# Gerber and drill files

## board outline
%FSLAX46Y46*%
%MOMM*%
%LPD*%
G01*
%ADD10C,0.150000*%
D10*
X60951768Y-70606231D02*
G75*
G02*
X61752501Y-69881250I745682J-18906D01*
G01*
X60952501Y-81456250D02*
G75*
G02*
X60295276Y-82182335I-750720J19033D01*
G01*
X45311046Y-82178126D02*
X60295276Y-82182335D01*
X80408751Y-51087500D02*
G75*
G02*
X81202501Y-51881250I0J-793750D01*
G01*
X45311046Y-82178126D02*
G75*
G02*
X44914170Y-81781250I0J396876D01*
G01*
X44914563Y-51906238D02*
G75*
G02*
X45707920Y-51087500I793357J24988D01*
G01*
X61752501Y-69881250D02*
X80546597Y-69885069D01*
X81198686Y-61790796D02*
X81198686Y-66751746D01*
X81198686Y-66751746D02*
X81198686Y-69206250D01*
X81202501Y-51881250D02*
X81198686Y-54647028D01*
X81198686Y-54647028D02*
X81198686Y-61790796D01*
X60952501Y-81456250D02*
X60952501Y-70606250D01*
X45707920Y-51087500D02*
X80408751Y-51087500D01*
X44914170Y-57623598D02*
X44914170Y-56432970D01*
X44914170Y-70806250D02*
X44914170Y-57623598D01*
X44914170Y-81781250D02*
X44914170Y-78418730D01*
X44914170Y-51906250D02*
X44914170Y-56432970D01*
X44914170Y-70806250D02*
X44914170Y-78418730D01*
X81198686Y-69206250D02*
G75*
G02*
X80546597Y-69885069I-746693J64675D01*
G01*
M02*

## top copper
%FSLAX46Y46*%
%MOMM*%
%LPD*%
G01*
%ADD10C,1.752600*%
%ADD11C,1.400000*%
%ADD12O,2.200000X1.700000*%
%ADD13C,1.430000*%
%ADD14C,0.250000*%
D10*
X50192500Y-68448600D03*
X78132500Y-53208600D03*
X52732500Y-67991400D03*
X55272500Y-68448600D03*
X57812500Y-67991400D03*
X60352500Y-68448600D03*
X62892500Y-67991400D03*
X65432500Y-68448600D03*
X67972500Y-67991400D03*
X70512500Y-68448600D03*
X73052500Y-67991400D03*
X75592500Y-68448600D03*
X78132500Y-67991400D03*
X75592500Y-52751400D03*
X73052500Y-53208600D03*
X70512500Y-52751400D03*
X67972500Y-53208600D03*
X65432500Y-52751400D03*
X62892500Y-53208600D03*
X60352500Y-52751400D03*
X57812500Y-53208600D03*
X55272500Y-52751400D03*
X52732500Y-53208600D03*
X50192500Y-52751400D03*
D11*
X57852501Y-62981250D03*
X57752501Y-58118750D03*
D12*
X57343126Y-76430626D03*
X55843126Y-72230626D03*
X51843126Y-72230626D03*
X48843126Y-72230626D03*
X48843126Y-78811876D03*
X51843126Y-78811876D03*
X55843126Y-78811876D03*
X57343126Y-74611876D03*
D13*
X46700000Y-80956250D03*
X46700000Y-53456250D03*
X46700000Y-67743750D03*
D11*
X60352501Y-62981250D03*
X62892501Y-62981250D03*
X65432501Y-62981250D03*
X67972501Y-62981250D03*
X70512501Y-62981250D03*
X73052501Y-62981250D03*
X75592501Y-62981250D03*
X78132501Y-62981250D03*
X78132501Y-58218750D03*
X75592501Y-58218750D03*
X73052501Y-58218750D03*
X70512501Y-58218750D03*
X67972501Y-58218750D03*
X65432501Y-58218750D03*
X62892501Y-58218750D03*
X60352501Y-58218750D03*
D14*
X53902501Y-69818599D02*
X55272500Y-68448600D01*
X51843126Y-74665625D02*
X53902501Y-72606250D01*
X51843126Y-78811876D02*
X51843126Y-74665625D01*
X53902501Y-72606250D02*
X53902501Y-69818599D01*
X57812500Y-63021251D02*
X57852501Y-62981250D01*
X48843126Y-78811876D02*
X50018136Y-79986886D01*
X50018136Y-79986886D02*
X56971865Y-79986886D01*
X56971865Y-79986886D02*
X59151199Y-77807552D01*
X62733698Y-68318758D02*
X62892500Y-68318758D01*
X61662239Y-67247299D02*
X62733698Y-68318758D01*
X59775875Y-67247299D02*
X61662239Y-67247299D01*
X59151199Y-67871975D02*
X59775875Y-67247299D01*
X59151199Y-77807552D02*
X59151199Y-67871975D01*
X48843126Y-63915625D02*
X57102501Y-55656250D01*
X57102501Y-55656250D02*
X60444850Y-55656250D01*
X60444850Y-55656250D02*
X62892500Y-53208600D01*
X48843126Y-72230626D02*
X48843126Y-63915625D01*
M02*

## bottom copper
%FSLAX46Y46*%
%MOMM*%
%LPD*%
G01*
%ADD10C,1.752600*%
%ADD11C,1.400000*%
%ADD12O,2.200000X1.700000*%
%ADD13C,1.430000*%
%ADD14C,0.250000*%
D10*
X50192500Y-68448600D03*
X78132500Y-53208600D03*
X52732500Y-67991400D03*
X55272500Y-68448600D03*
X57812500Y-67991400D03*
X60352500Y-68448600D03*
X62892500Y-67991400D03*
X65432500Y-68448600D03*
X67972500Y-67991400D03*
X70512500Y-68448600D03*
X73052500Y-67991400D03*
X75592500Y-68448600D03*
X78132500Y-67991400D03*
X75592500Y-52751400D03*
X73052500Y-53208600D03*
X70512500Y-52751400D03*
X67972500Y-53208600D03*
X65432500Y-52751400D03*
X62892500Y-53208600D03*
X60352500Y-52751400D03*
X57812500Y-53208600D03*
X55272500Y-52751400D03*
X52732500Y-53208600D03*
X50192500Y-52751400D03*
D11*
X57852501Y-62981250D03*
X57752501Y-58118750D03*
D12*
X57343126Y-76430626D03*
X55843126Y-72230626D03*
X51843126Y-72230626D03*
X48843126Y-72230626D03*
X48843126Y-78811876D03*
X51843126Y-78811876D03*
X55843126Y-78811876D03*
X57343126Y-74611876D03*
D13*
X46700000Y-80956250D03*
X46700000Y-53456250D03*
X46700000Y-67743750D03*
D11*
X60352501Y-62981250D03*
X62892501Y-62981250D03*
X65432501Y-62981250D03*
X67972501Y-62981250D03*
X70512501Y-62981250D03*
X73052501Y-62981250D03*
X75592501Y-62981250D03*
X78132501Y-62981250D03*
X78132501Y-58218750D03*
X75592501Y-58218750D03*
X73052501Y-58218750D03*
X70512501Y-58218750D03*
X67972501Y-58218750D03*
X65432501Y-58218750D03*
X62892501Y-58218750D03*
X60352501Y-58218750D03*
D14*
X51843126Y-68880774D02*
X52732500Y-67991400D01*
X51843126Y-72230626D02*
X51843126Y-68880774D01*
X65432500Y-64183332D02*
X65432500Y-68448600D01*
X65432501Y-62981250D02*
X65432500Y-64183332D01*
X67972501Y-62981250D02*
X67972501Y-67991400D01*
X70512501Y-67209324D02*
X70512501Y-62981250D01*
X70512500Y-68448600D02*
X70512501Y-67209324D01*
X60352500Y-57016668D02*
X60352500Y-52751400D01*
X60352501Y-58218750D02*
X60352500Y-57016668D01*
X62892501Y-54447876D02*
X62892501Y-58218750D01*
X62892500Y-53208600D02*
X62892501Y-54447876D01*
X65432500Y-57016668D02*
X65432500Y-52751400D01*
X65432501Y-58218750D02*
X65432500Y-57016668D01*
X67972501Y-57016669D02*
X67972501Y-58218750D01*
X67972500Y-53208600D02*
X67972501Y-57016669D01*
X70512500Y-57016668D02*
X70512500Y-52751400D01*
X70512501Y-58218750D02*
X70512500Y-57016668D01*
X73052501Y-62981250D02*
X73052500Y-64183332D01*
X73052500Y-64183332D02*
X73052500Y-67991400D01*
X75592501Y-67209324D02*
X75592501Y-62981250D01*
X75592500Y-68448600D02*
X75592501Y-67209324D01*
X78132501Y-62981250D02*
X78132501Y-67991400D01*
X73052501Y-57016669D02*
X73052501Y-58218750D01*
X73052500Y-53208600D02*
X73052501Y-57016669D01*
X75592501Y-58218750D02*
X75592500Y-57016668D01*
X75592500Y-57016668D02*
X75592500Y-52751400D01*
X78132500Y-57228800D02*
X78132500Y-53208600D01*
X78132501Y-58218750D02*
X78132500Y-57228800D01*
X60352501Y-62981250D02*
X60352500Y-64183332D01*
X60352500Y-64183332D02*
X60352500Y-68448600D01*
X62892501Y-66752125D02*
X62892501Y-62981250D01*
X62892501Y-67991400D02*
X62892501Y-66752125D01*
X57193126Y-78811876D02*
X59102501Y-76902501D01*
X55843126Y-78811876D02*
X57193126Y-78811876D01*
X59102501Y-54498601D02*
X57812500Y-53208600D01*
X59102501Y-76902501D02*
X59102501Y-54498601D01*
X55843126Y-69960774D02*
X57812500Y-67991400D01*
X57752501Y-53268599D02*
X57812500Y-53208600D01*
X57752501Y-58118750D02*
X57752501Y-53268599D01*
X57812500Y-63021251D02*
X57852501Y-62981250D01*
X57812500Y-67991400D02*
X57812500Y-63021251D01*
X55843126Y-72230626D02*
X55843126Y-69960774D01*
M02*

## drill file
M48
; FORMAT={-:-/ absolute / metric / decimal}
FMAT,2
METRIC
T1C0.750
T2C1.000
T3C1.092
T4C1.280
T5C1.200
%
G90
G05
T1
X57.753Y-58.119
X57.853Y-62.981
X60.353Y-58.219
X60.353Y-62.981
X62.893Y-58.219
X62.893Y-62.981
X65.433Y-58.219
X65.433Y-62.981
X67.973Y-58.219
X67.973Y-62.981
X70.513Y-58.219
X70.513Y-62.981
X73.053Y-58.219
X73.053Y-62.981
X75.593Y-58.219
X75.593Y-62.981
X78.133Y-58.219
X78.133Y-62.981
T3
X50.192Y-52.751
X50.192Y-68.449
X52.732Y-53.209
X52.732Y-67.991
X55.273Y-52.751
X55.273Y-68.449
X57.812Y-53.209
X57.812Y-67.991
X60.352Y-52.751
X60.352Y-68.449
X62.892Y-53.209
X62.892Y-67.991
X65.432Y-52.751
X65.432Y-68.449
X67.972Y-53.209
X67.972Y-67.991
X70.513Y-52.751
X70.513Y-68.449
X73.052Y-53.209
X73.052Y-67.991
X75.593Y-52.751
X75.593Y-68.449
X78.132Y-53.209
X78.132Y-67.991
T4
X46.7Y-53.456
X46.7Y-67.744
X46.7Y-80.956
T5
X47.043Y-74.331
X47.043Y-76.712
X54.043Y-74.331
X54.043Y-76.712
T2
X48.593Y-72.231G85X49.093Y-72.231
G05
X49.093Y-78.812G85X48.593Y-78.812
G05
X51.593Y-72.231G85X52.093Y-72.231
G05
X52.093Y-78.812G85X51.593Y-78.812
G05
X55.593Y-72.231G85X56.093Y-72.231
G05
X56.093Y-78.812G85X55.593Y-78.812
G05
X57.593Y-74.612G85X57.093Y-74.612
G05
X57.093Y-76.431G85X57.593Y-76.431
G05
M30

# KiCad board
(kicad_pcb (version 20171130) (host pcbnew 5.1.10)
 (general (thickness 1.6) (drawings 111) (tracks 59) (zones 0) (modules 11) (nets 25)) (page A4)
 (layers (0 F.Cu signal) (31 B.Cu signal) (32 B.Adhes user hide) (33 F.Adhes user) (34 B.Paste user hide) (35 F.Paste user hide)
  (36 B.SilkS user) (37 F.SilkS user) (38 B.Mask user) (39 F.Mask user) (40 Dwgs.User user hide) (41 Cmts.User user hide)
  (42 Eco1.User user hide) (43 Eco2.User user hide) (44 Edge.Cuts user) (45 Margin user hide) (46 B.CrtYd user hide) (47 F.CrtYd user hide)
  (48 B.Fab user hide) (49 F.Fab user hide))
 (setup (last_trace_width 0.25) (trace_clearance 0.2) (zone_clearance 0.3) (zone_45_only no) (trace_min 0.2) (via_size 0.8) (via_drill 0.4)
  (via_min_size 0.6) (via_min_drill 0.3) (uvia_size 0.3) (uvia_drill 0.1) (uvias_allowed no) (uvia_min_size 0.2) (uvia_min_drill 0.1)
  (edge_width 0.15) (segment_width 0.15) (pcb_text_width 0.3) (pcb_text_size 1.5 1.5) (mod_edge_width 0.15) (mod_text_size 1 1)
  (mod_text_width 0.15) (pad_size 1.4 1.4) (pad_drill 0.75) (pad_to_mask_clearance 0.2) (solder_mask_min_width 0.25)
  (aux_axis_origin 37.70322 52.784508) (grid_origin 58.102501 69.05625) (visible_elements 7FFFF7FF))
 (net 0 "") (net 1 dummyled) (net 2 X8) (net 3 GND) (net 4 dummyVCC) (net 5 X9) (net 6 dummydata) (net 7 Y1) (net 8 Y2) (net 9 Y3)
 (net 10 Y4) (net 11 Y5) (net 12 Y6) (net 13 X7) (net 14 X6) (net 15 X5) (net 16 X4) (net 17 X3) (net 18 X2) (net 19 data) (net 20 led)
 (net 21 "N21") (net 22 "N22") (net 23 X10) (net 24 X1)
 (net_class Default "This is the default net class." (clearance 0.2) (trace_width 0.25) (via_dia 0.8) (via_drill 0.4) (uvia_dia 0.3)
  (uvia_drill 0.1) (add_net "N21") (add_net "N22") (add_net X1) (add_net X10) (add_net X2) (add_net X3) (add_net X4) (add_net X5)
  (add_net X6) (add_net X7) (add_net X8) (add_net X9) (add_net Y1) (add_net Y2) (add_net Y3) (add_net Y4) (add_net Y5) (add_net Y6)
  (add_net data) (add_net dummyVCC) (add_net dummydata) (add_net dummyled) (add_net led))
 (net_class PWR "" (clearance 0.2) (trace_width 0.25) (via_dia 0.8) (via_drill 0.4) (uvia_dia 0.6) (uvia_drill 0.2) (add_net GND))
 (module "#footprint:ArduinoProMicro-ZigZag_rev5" (layer B.Cu) (at 64.1625 60.6)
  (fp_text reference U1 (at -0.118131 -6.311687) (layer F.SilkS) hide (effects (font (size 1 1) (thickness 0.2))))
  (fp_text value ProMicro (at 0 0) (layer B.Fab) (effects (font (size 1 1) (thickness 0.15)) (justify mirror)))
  (pad 24 thru_hole circle (at -13.97 7.8486) (size 1.7526 1.7526) (drill 1.0922) (layers *.Cu *.SilkS *.Mask) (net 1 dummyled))
  (pad 12 thru_hole circle (at 13.97 -7.3914) (size 1.7526 1.7526) (drill 1.0922) (layers *.Cu *.SilkS *.Mask) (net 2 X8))
  (pad 23 thru_hole circle (at -11.43 7.3914) (size 1.7526 1.7526) (drill 1.0922) (layers *.Cu *.SilkS *.Mask) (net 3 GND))
  (pad 22 thru_hole circle (at -8.89 7.8486) (size 1.7526 1.7526) (drill 1.0922) (layers *.Cu *.SilkS *.Mask) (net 3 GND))
  (pad 21 thru_hole circle (at -6.35 7.3914) (size 1.7526 1.7526) (drill 1.0922) (layers *.Cu *.SilkS *.Mask) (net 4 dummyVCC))
  (pad 20 thru_hole circle (at -3.81 7.8486) (size 1.7526 1.7526) (drill 1.0922) (layers *.Cu *.SilkS *.Mask) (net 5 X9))
  (pad 19 thru_hole circle (at -1.27 7.3914) (size 1.7526 1.7526) (drill 1.0922) (layers *.Cu *.SilkS *.Mask) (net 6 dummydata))
  (pad 18 thru_hole circle (at 1.27 7.8486) (size 1.7526 1.7526) (drill 1.0922) (layers *.Cu *.SilkS *.Mask) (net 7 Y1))
  (pad 17 thru_hole circle (at 3.81 7.3914) (size 1.7526 1.7526) (drill 1.0922) (layers *.Cu *.SilkS *.Mask) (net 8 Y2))
  (pad 16 thru_hole circle (at 6.35 7.8486) (size 1.7526 1.7526) (drill 1.0922) (layers *.Cu *.SilkS *.Mask) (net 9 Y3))
  (pad 15 thru_hole circle (at 8.89 7.3914) (size 1.7526 1.7526) (drill 1.0922) (layers *.Cu *.SilkS *.Mask) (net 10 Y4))
  (pad 14 thru_hole circle (at 11.43 7.8486) (size 1.7526 1.7526) (drill 1.0922) (layers *.Cu *.SilkS *.Mask) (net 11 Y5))
  (pad 13 thru_hole circle (at 13.97 7.3914) (size 1.7526 1.7526) (drill 1.0922) (layers *.Cu *.SilkS *.Mask) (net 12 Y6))
  (pad 11 thru_hole circle (at 11.43 -7.8486) (size 1.7526 1.7526) (drill 1.0922) (layers *.Cu *.SilkS *.Mask) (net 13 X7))
  (pad 10 thru_hole circle (at 8.89 -7.3914) (size 1.7526 1.7526) (drill 1.0922) (layers *.Cu *.SilkS *.Mask) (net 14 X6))
  (pad 9 thru_hole circle (at 6.35 -7.8486) (size 1.7526 1.7526) (drill 1.0922) (layers *.Cu *.SilkS *.Mask) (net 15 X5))
  (pad 8 thru_hole circle (at 3.81 -7.3914) (size 1.7526 1.7526) (drill 1.0922) (layers *.Cu *.SilkS *.Mask) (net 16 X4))
  (pad 7 thru_hole circle (at 1.27 -7.8486) (size 1.7526 1.7526) (drill 1.0922) (layers *.Cu *.SilkS *.Mask) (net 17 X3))
  (pad 6 thru_hole circle (at -1.27 -7.3914) (size 1.7526 1.7526) (drill 1.0922) (layers *.Cu *.SilkS *.Mask) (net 6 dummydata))
  (pad 5 thru_hole circle (at -3.81 -7.8486) (size 1.7526 1.7526) (drill 1.0922) (layers *.Cu *.SilkS *.Mask) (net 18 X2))
  (pad 4 thru_hole circle (at -6.35 -7.3914) (size 1.7526 1.7526) (drill 1.0922) (layers *.Cu *.SilkS *.Mask) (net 4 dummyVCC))
  (pad 3 thru_hole circle (at -8.89 -7.8486) (size 1.7526 1.7526) (drill 1.0922) (layers *.Cu *.SilkS *.Mask) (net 3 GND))
  (pad 2 thru_hole circle (at -11.43 -7.3914) (size 1.7526 1.7526) (drill 1.0922) (layers *.Cu *.SilkS *.Mask) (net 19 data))
  (pad 1 thru_hole circle (at -13.97 -7.8486) (size 1.7526 1.7526) (drill 1.0922) (layers *.Cu *.SilkS *.Mask) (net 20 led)))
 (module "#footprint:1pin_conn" (layer F.Cu) (at 57.852501 63.00625) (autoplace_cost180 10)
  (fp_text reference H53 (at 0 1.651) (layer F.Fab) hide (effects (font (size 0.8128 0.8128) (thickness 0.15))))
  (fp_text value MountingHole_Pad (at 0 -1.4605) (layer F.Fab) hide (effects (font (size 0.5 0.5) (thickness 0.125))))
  (pad 1 thru_hole circle (at 0 -0.025) (size 1.4 1.4) (drill 0.75) (layers *.Cu *.Mask) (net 4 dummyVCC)))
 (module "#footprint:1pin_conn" (layer F.Cu) (at 57.752501 58.21875) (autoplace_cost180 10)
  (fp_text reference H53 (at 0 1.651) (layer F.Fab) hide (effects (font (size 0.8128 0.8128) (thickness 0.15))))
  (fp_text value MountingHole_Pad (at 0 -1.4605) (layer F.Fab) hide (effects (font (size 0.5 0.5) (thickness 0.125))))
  (pad 1 thru_hole circle (at 0 -0.1) (size 1.4 1.4) (drill 0.75) (layers *.Cu *.Mask) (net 4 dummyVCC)))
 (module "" (layer F.Cu) (at 7.352501 -16.34375)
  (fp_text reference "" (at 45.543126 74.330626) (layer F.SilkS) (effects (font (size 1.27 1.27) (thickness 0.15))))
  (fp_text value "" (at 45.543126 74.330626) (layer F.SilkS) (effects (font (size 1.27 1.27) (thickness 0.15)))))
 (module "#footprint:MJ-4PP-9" (layer F.Cu) (at 45.543126 74.330626 90)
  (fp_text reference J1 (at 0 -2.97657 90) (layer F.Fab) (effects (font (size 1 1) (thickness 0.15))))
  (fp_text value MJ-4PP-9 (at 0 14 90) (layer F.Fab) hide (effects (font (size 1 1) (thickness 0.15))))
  (pad A thru_hole oval (at -2.1 11.8 90) (size 1.7 2.2) (drill oval 1 1.5) (layers *.Cu *.Mask F.SilkS) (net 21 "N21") (clearance 0.15))
  (pad D thru_hole oval (at 2.1 10.3 90) (size 1.7 2.2) (drill oval 1 1.5) (layers *.Cu *.Mask F.SilkS) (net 4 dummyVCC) (clearance 0.15))
  (pad C thru_hole oval (at 2.1 6.3 90) (size 1.7 2.2) (drill oval 1 1.5) (layers *.Cu *.Mask F.SilkS) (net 3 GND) (clearance 0.15))
  (pad B thru_hole oval (at 2.1 3.3 90) (size 1.7 2.2) (drill oval 1 1.5) (layers *.Cu *.Mask F.SilkS) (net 6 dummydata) (clearance 0.15))
  (pad "" np_thru_hole circle (at 0 8.5 90) (size 1.2 1.2) (drill 1.2) (layers *.Cu *.Mask F.SilkS))
  (pad "" np_thru_hole circle (at 0 1.5 90) (size 1.2 1.2) (drill 1.2) (layers *.Cu *.Mask F.SilkS)))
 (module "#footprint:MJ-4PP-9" (layer B.Cu) (at 45.543126 76.711876 270)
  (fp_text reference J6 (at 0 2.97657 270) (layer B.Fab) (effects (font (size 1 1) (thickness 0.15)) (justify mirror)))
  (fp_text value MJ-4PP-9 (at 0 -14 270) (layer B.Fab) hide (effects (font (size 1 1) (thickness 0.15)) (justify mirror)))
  (pad "" np_thru_hole circle (at 0 -1.5 270) (size 1.2 1.2) (drill 1.2) (layers *.Cu *.Mask B.SilkS))
  (pad "" np_thru_hole circle (at 0 -8.5 270) (size 1.2 1.2) (drill 1.2) (layers *.Cu *.Mask B.SilkS))
  (pad B thru_hole oval (at 2.1 -3.3 270) (size 1.7 2.2) (drill oval 1 1.5) (layers *.Cu *.Mask B.SilkS) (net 6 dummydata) (clearance 0.15))
  (pad C thru_hole oval (at 2.1 -6.3 270) (size 1.7 2.2) (drill oval 1 1.5) (layers *.Cu *.Mask B.SilkS) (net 3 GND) (clearance 0.15))
  (pad D thru_hole oval (at 2.1 -10.3 270) (size 1.7 2.2) (drill oval 1 1.5) (layers *.Cu *.Mask B.SilkS) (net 4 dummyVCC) (clearance 0.15))
  (pad A thru_hole oval (at -2.1 -11.8 270) (size 1.7 2.2) (drill oval 1 1.5) (layers *.Cu *.Mask B.SilkS) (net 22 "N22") (clearance 0.15)))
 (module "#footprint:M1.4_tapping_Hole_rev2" (layer F.Cu) (at 46.102501 80.95625) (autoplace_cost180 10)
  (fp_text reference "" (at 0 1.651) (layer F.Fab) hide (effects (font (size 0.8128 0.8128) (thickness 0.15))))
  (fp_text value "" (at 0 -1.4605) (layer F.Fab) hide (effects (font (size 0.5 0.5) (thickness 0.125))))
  (pad "" thru_hole circle (at 0.597499 0) (size 1.43 1.43) (drill 1.28) (layers *.Cu *.Mask)))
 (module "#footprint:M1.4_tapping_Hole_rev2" (layer F.Cu) (at 46.7 53.45625) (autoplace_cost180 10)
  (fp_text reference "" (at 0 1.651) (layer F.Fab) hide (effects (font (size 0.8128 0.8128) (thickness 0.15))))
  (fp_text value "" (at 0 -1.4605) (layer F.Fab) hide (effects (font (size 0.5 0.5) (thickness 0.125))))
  (pad "" thru_hole circle (at 0 0) (size 1.43 1.43) (drill 1.28) (layers *.Cu *.Mask)))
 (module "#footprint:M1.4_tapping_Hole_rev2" (layer F.Cu) (at 46.7 67.74375) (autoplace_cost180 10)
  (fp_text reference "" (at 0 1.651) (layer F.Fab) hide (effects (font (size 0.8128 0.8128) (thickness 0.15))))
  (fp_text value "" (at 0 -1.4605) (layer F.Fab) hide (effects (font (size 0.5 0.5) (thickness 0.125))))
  (pad "" thru_hole circle (at 0 0) (size 1.43 1.43) (drill 1.28) (layers *.Cu *.Mask)))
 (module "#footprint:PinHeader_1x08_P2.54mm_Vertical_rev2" (layer F.Cu) (at 60.352501 62.98125 90)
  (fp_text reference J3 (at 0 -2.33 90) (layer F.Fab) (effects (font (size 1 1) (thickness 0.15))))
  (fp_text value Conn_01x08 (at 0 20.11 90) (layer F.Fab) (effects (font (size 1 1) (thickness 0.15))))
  (pad 1 thru_hole circle (at 0 0 90) (size 1.4 1.4) (drill 0.75) (layers *.Cu *.Mask) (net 5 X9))
  (pad 2 thru_hole circle (at 0 2.54 90) (size 1.4 1.4) (drill 0.75) (layers *.Cu *.Mask) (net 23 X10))
  (pad 3 thru_hole circle (at 0 5.08 90) (size 1.4 1.4) (drill 0.75) (layers *.Cu *.Mask) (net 7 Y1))
  (pad 4 thru_hole circle (at 0 7.62 90) (size 1.4 1.4) (drill 0.75) (layers *.Cu *.Mask) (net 8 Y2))
  (pad 5 thru_hole circle (at 0 10.16 90) (size 1.4 1.4) (drill 0.75) (layers *.Cu *.Mask) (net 9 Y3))
  (pad 6 thru_hole circle (at 0 12.7 90) (size 1.4 1.4) (drill 0.75) (layers *.Cu *.Mask) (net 10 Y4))
  (pad 7 thru_hole circle (at 0 15.24 90) (size 1.4 1.4) (drill 0.75) (layers *.Cu *.Mask) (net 11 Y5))
  (pad 8 thru_hole circle (at 0 17.78 90) (size 1.4 1.4) (drill 0.75) (layers *.Cu *.Mask) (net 12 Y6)))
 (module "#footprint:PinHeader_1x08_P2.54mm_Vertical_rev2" (layer F.Cu) (at 60.352501 58.21875 90)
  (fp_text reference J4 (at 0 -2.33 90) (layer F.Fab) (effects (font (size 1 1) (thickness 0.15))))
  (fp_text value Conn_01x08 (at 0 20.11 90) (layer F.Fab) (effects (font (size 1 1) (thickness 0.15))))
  (pad 8 thru_hole circle (at 0 17.78 90) (size 1.4 1.4) (drill 0.75) (layers *.Cu *.Mask) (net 2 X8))
  (pad 7 thru_hole circle (at 0 15.24 90) (size 1.4 1.4) (drill 0.75) (layers *.Cu *.Mask) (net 13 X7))
  (pad 6 thru_hole circle (at 0 12.7 90) (size 1.4 1.4) (drill 0.75) (layers *.Cu *.Mask) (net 14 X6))
  (pad 5 thru_hole circle (at 0 10.16 90) (size 1.4 1.4) (drill 0.75) (layers *.Cu *.Mask) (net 15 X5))
  (pad 4 thru_hole circle (at 0 7.62 90) (size 1.4 1.4) (drill 0.75) (layers *.Cu *.Mask) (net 16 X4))
  (pad 3 thru_hole circle (at 0 5.08 90) (size 1.4 1.4) (drill 0.75) (layers *.Cu *.Mask) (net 17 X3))
  (pad 2 thru_hole circle (at 0 2.54 90) (size 1.4 1.4) (drill 0.75) (layers *.Cu *.Mask) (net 18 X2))
  (pad 1 thru_hole circle (at 0 0 90) (size 1.4 1.4) (drill 0.75) (layers *.Cu *.Mask) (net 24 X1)))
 (gr_arc (start 61.69745 70.625137) (end 61.752501 69.88125) (angle -92.78006695) (layer Edge.Cuts) (width 0.15))
 (gr_arc (start 60.201781 81.437217) (end 60.295276 82.182335) (angle -81.39578011) (layer Edge.Cuts) (width 0.15))
 (gr_line (start 45.311046 82.178126) (end 60.295276 82.182335) (layer Edge.Cuts) (width 0.15))
 (gr_arc (start 80.408751 51.88125) (end 81.202501 51.88125) (angle -90) (layer Edge.Cuts) (width 0.15))
 (gr_arc (start 45.311046 81.78125) (end 44.91417 81.78125) (angle -90) (layer Edge.Cuts) (width 0.15))
 (gr_arc (start 45.70792 51.88125) (end 45.70792 51.0875) (angle -91.80399512) (layer Edge.Cuts) (width 0.15))
 (gr_line (start 61.752501 69.88125) (end 80.546597 69.885069) (layer Edge.Cuts) (width 0.15))
 (gr_line (start 81.198686 61.790796) (end 81.198686 66.751746) (layer Edge.Cuts) (width 0.15))
 (gr_line (start 81.198686 66.751746) (end 81.198686 69.20625) (layer Edge.Cuts) (width 0.15))
 (gr_line (start 81.202501 51.88125) (end 81.198686 54.647028) (layer Edge.Cuts) (width 0.15))
 (gr_line (start 81.198686 54.647028) (end 81.198686 61.790796) (layer Edge.Cuts) (width 0.15))
 (gr_line (start 60.952501 81.45625) (end 60.952501 70.60625) (layer Edge.Cuts) (width 0.15))
 (gr_line (start 45.70792 51.0875) (end 80.408751 51.0875) (layer Edge.Cuts) (width 0.15))
 (gr_line (start 44.91417 57.623598) (end 44.91417 56.43297) (layer Edge.Cuts) (width 0.15))
 (gr_line (start 44.91417 70.80625) (end 44.91417 57.623598) (layer Edge.Cuts) (width 0.15))
 (gr_line (start 44.91417 81.78125) (end 44.91417 78.41873) (layer Edge.Cuts) (width 0.15))
 (gr_line (start 44.91417 51.90625) (end 44.91417 56.43297) (layer Edge.Cuts) (width 0.15))
 (gr_line (start 44.91417 70.80625) (end 44.91417 78.41873) (layer Edge.Cuts) (width 0.15))
 (gr_arc (start 80.451993 69.141575) (end 80.546597 69.885069) (angle -77.79817896) (layer Edge.Cuts) (width 0.15))
 (segment (start 53.902501 69.818599) (end 55.2725 68.4486) (width 0.25) (layer F.Cu) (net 3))
 (segment (start 51.843126 74.665625) (end 53.902501 72.60625) (width 0.25) (layer F.Cu) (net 3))
 (segment (start 51.843126 78.811876) (end 51.843126 74.665625) (width 0.25) (layer F.Cu) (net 3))
 (segment (start 51.843126 68.880774) (end 52.7325 67.9914) (width 0.25) (layer B.Cu) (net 3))
 (segment (start 51.843126 72.230626) (end 51.843126 68.880774) (width 0.25) (layer B.Cu) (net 3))
 (segment (start 53.902501 72.60625) (end 53.902501 69.818599) (width 0.25) (layer F.Cu) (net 3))
 (segment (start 65.4325 64.183332) (end 65.4325 68.4486) (width 0.25) (layer B.Cu) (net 7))
 (segment (start 65.432501 62.98125) (end 65.4325 64.183332) (width 0.25) (layer B.Cu) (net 7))
 (segment (start 67.972501 62.98125) (end 67.972501 67.9914) (width 0.25) (layer B.Cu) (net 8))
 (segment (start 70.512501 67.209324) (end 70.512501 62.98125) (width 0.25) (layer B.Cu) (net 9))
 (segment (start 70.5125 68.4486) (end 70.512501 67.209324) (width 0.25) (layer B.Cu) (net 9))
 (segment (start 60.3525 57.016668) (end 60.3525 52.7514) (width 0.25) (layer B.Cu) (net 24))
 (segment (start 60.352501 58.21875) (end 60.3525 57.016668) (width 0.25) (layer B.Cu) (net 24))
 (segment (start 62.892501 54.447876) (end 62.892501 58.21875) (width 0.25) (layer B.Cu) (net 18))
 (segment (start 62.8925 53.2086) (end 62.892501 54.447876) (width 0.25) (layer B.Cu) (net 18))
 (segment (start 65.4325 57.016668) (end 65.4325 52.7514) (width 0.25) (layer B.Cu) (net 17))
 (segment (start 65.432501 58.21875) (end 65.4325 57.016668) (width 0.25) (layer B.Cu) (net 17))
 (segment (start 67.972501 57.016669) (end 67.972501 58.21875) (width 0.25) (layer B.Cu) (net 16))
 (segment (start 67.9725 53.2086) (end 67.972501 57.016669) (width 0.25) (layer B.Cu) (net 16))
 (segment (start 70.5125 57.016668) (end 70.5125 52.7514) (width 0.25) (layer B.Cu) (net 15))
 (segment (start 70.512501 58.21875) (end 70.5125 57.016668) (width 0.25) (layer B.Cu) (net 15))
 (segment (start 73.052501 62.98125) (end 73.0525 64.183332) (width 0.25) (layer B.Cu) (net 10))
 (segment (start 73.0525 64.183332) (end 73.0525 67.9914) (width 0.25) (layer B.Cu) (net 10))
 (segment (start 75.592501 67.209324) (end 75.592501 62.98125) (width 0.25) (layer B.Cu) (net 11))
 (segment (start 75.5925 68.4486) (end 75.592501 67.209324) (width 0.25) (layer B.Cu) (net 11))
 (segment (start 78.132501 62.98125) (end 78.132501 67.9914) (width 0.25) (layer B.Cu) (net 12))
 (segment (start 73.052501 57.016669) (end 73.052501 58.21875) (width 0.25) (layer B.Cu) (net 14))
 (segment (start 73.0525 53.2086) (end 73.052501 57.016669) (width 0.25) (layer B.Cu) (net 14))
 (segment (start 75.592501 58.21875) (end 75.5925 57.016668) (width 0.25) (layer B.Cu) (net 13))
 (segment (start 75.5925 57.016668) (end 75.5925 52.7514) (width 0.25) (layer B.Cu) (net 13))
 (segment (start 78.1325 57.2288) (end 78.1325 53.2086) (width 0.25) (layer B.Cu) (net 2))
 (segment (start 78.132501 58.21875) (end 78.1325 57.2288) (width 0.25) (layer B.Cu) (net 2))
 (segment (start 60.352501 62.98125) (end 60.3525 64.183332) (width 0.25) (layer B.Cu) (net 5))
 (segment (start 60.3525 64.183332) (end 60.3525 68.4486) (width 0.25) (layer B.Cu) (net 5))
 (segment (start 62.892501 66.752125) (end 62.892501 62.98125) (width 0.25) (layer B.Cu) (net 23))
 (segment (start 62.892501 67.9914) (end 62.892501 66.752125) (width 0.25) (layer B.Cu) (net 23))
 (segment (start 57.193126 78.811876) (end 59.102501 76.902501) (width 0.25) (layer B.Cu) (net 4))
 (segment (start 55.843126 78.811876) (end 57.193126 78.811876) (width 0.25) (layer B.Cu) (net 4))
 (segment (start 59.102501 54.498601) (end 57.8125 53.2086) (width 0.25) (layer B.Cu) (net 4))
 (segment (start 59.102501 76.902501) (end 59.102501 54.498601) (width 0.25) (layer B.Cu) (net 4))
 (segment (start 55.843126 69.960774) (end 57.8125 67.9914) (width 0.25) (layer B.Cu) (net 4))
 (segment (start 57.752501 53.268599) (end 57.8125 53.2086) (width 0.25) (layer B.Cu) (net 4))
 (segment (start 57.752501 58.11875) (end 57.752501 53.268599) (width 0.25) (layer B.Cu) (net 4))
 (segment (start 57.8125 63.021251) (end 57.852501 62.98125) (width 0.25) (layer F.Cu) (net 4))
 (segment (start 57.8125 63.021251) (end 57.852501 62.98125) (width 0.25) (layer B.Cu) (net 4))
 (segment (start 57.8125 67.9914) (end 57.8125 63.021251) (width 0.25) (layer B.Cu) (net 4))
 (segment (start 55.843126 72.230626) (end 55.843126 69.960774) (width 0.25) (layer B.Cu) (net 4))
 (segment (start 48.843126 78.811876) (end 50.018136 79.986886) (width 0.25) (layer F.Cu) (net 6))
 (segment (start 50.018136 79.986886) (end 56.971865 79.986886) (width 0.25) (layer F.Cu) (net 6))
 (segment (start 56.971865 79.986886) (end 59.151199 77.807552) (width 0.25) (layer F.Cu) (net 6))
 (segment (start 62.733698 68.318758) (end 62.8925 68.318758) (width 0.25) (layer F.Cu) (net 6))
 (segment (start 61.662239 67.247299) (end 62.733698 68.318758) (width 0.25) (layer F.Cu) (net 6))
 (segment (start 59.775875 67.247299) (end 61.662239 67.247299) (width 0.25) (layer F.Cu) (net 6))
 (segment (start 59.151199 67.871975) (end 59.775875 67.247299) (width 0.25) (layer F.Cu) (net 6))
 (segment (start 59.151199 77.807552) (end 59.151199 67.871975) (width 0.25) (layer F.Cu) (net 6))
 (segment (start 48.843126 63.915625) (end 57.102501 55.65625) (width 0.25) (layer F.Cu) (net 6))
 (segment (start 57.102501 55.65625) (end 60.44485 55.65625) (width 0.25) (layer F.Cu) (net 6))
 (segment (start 60.44485 55.65625) (end 62.8925 53.2086) (width 0.25) (layer F.Cu) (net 6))
 (segment (start 48.843126 72.230626) (end 48.843126 63.915625) (width 0.25) (layer F.Cu) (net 6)))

